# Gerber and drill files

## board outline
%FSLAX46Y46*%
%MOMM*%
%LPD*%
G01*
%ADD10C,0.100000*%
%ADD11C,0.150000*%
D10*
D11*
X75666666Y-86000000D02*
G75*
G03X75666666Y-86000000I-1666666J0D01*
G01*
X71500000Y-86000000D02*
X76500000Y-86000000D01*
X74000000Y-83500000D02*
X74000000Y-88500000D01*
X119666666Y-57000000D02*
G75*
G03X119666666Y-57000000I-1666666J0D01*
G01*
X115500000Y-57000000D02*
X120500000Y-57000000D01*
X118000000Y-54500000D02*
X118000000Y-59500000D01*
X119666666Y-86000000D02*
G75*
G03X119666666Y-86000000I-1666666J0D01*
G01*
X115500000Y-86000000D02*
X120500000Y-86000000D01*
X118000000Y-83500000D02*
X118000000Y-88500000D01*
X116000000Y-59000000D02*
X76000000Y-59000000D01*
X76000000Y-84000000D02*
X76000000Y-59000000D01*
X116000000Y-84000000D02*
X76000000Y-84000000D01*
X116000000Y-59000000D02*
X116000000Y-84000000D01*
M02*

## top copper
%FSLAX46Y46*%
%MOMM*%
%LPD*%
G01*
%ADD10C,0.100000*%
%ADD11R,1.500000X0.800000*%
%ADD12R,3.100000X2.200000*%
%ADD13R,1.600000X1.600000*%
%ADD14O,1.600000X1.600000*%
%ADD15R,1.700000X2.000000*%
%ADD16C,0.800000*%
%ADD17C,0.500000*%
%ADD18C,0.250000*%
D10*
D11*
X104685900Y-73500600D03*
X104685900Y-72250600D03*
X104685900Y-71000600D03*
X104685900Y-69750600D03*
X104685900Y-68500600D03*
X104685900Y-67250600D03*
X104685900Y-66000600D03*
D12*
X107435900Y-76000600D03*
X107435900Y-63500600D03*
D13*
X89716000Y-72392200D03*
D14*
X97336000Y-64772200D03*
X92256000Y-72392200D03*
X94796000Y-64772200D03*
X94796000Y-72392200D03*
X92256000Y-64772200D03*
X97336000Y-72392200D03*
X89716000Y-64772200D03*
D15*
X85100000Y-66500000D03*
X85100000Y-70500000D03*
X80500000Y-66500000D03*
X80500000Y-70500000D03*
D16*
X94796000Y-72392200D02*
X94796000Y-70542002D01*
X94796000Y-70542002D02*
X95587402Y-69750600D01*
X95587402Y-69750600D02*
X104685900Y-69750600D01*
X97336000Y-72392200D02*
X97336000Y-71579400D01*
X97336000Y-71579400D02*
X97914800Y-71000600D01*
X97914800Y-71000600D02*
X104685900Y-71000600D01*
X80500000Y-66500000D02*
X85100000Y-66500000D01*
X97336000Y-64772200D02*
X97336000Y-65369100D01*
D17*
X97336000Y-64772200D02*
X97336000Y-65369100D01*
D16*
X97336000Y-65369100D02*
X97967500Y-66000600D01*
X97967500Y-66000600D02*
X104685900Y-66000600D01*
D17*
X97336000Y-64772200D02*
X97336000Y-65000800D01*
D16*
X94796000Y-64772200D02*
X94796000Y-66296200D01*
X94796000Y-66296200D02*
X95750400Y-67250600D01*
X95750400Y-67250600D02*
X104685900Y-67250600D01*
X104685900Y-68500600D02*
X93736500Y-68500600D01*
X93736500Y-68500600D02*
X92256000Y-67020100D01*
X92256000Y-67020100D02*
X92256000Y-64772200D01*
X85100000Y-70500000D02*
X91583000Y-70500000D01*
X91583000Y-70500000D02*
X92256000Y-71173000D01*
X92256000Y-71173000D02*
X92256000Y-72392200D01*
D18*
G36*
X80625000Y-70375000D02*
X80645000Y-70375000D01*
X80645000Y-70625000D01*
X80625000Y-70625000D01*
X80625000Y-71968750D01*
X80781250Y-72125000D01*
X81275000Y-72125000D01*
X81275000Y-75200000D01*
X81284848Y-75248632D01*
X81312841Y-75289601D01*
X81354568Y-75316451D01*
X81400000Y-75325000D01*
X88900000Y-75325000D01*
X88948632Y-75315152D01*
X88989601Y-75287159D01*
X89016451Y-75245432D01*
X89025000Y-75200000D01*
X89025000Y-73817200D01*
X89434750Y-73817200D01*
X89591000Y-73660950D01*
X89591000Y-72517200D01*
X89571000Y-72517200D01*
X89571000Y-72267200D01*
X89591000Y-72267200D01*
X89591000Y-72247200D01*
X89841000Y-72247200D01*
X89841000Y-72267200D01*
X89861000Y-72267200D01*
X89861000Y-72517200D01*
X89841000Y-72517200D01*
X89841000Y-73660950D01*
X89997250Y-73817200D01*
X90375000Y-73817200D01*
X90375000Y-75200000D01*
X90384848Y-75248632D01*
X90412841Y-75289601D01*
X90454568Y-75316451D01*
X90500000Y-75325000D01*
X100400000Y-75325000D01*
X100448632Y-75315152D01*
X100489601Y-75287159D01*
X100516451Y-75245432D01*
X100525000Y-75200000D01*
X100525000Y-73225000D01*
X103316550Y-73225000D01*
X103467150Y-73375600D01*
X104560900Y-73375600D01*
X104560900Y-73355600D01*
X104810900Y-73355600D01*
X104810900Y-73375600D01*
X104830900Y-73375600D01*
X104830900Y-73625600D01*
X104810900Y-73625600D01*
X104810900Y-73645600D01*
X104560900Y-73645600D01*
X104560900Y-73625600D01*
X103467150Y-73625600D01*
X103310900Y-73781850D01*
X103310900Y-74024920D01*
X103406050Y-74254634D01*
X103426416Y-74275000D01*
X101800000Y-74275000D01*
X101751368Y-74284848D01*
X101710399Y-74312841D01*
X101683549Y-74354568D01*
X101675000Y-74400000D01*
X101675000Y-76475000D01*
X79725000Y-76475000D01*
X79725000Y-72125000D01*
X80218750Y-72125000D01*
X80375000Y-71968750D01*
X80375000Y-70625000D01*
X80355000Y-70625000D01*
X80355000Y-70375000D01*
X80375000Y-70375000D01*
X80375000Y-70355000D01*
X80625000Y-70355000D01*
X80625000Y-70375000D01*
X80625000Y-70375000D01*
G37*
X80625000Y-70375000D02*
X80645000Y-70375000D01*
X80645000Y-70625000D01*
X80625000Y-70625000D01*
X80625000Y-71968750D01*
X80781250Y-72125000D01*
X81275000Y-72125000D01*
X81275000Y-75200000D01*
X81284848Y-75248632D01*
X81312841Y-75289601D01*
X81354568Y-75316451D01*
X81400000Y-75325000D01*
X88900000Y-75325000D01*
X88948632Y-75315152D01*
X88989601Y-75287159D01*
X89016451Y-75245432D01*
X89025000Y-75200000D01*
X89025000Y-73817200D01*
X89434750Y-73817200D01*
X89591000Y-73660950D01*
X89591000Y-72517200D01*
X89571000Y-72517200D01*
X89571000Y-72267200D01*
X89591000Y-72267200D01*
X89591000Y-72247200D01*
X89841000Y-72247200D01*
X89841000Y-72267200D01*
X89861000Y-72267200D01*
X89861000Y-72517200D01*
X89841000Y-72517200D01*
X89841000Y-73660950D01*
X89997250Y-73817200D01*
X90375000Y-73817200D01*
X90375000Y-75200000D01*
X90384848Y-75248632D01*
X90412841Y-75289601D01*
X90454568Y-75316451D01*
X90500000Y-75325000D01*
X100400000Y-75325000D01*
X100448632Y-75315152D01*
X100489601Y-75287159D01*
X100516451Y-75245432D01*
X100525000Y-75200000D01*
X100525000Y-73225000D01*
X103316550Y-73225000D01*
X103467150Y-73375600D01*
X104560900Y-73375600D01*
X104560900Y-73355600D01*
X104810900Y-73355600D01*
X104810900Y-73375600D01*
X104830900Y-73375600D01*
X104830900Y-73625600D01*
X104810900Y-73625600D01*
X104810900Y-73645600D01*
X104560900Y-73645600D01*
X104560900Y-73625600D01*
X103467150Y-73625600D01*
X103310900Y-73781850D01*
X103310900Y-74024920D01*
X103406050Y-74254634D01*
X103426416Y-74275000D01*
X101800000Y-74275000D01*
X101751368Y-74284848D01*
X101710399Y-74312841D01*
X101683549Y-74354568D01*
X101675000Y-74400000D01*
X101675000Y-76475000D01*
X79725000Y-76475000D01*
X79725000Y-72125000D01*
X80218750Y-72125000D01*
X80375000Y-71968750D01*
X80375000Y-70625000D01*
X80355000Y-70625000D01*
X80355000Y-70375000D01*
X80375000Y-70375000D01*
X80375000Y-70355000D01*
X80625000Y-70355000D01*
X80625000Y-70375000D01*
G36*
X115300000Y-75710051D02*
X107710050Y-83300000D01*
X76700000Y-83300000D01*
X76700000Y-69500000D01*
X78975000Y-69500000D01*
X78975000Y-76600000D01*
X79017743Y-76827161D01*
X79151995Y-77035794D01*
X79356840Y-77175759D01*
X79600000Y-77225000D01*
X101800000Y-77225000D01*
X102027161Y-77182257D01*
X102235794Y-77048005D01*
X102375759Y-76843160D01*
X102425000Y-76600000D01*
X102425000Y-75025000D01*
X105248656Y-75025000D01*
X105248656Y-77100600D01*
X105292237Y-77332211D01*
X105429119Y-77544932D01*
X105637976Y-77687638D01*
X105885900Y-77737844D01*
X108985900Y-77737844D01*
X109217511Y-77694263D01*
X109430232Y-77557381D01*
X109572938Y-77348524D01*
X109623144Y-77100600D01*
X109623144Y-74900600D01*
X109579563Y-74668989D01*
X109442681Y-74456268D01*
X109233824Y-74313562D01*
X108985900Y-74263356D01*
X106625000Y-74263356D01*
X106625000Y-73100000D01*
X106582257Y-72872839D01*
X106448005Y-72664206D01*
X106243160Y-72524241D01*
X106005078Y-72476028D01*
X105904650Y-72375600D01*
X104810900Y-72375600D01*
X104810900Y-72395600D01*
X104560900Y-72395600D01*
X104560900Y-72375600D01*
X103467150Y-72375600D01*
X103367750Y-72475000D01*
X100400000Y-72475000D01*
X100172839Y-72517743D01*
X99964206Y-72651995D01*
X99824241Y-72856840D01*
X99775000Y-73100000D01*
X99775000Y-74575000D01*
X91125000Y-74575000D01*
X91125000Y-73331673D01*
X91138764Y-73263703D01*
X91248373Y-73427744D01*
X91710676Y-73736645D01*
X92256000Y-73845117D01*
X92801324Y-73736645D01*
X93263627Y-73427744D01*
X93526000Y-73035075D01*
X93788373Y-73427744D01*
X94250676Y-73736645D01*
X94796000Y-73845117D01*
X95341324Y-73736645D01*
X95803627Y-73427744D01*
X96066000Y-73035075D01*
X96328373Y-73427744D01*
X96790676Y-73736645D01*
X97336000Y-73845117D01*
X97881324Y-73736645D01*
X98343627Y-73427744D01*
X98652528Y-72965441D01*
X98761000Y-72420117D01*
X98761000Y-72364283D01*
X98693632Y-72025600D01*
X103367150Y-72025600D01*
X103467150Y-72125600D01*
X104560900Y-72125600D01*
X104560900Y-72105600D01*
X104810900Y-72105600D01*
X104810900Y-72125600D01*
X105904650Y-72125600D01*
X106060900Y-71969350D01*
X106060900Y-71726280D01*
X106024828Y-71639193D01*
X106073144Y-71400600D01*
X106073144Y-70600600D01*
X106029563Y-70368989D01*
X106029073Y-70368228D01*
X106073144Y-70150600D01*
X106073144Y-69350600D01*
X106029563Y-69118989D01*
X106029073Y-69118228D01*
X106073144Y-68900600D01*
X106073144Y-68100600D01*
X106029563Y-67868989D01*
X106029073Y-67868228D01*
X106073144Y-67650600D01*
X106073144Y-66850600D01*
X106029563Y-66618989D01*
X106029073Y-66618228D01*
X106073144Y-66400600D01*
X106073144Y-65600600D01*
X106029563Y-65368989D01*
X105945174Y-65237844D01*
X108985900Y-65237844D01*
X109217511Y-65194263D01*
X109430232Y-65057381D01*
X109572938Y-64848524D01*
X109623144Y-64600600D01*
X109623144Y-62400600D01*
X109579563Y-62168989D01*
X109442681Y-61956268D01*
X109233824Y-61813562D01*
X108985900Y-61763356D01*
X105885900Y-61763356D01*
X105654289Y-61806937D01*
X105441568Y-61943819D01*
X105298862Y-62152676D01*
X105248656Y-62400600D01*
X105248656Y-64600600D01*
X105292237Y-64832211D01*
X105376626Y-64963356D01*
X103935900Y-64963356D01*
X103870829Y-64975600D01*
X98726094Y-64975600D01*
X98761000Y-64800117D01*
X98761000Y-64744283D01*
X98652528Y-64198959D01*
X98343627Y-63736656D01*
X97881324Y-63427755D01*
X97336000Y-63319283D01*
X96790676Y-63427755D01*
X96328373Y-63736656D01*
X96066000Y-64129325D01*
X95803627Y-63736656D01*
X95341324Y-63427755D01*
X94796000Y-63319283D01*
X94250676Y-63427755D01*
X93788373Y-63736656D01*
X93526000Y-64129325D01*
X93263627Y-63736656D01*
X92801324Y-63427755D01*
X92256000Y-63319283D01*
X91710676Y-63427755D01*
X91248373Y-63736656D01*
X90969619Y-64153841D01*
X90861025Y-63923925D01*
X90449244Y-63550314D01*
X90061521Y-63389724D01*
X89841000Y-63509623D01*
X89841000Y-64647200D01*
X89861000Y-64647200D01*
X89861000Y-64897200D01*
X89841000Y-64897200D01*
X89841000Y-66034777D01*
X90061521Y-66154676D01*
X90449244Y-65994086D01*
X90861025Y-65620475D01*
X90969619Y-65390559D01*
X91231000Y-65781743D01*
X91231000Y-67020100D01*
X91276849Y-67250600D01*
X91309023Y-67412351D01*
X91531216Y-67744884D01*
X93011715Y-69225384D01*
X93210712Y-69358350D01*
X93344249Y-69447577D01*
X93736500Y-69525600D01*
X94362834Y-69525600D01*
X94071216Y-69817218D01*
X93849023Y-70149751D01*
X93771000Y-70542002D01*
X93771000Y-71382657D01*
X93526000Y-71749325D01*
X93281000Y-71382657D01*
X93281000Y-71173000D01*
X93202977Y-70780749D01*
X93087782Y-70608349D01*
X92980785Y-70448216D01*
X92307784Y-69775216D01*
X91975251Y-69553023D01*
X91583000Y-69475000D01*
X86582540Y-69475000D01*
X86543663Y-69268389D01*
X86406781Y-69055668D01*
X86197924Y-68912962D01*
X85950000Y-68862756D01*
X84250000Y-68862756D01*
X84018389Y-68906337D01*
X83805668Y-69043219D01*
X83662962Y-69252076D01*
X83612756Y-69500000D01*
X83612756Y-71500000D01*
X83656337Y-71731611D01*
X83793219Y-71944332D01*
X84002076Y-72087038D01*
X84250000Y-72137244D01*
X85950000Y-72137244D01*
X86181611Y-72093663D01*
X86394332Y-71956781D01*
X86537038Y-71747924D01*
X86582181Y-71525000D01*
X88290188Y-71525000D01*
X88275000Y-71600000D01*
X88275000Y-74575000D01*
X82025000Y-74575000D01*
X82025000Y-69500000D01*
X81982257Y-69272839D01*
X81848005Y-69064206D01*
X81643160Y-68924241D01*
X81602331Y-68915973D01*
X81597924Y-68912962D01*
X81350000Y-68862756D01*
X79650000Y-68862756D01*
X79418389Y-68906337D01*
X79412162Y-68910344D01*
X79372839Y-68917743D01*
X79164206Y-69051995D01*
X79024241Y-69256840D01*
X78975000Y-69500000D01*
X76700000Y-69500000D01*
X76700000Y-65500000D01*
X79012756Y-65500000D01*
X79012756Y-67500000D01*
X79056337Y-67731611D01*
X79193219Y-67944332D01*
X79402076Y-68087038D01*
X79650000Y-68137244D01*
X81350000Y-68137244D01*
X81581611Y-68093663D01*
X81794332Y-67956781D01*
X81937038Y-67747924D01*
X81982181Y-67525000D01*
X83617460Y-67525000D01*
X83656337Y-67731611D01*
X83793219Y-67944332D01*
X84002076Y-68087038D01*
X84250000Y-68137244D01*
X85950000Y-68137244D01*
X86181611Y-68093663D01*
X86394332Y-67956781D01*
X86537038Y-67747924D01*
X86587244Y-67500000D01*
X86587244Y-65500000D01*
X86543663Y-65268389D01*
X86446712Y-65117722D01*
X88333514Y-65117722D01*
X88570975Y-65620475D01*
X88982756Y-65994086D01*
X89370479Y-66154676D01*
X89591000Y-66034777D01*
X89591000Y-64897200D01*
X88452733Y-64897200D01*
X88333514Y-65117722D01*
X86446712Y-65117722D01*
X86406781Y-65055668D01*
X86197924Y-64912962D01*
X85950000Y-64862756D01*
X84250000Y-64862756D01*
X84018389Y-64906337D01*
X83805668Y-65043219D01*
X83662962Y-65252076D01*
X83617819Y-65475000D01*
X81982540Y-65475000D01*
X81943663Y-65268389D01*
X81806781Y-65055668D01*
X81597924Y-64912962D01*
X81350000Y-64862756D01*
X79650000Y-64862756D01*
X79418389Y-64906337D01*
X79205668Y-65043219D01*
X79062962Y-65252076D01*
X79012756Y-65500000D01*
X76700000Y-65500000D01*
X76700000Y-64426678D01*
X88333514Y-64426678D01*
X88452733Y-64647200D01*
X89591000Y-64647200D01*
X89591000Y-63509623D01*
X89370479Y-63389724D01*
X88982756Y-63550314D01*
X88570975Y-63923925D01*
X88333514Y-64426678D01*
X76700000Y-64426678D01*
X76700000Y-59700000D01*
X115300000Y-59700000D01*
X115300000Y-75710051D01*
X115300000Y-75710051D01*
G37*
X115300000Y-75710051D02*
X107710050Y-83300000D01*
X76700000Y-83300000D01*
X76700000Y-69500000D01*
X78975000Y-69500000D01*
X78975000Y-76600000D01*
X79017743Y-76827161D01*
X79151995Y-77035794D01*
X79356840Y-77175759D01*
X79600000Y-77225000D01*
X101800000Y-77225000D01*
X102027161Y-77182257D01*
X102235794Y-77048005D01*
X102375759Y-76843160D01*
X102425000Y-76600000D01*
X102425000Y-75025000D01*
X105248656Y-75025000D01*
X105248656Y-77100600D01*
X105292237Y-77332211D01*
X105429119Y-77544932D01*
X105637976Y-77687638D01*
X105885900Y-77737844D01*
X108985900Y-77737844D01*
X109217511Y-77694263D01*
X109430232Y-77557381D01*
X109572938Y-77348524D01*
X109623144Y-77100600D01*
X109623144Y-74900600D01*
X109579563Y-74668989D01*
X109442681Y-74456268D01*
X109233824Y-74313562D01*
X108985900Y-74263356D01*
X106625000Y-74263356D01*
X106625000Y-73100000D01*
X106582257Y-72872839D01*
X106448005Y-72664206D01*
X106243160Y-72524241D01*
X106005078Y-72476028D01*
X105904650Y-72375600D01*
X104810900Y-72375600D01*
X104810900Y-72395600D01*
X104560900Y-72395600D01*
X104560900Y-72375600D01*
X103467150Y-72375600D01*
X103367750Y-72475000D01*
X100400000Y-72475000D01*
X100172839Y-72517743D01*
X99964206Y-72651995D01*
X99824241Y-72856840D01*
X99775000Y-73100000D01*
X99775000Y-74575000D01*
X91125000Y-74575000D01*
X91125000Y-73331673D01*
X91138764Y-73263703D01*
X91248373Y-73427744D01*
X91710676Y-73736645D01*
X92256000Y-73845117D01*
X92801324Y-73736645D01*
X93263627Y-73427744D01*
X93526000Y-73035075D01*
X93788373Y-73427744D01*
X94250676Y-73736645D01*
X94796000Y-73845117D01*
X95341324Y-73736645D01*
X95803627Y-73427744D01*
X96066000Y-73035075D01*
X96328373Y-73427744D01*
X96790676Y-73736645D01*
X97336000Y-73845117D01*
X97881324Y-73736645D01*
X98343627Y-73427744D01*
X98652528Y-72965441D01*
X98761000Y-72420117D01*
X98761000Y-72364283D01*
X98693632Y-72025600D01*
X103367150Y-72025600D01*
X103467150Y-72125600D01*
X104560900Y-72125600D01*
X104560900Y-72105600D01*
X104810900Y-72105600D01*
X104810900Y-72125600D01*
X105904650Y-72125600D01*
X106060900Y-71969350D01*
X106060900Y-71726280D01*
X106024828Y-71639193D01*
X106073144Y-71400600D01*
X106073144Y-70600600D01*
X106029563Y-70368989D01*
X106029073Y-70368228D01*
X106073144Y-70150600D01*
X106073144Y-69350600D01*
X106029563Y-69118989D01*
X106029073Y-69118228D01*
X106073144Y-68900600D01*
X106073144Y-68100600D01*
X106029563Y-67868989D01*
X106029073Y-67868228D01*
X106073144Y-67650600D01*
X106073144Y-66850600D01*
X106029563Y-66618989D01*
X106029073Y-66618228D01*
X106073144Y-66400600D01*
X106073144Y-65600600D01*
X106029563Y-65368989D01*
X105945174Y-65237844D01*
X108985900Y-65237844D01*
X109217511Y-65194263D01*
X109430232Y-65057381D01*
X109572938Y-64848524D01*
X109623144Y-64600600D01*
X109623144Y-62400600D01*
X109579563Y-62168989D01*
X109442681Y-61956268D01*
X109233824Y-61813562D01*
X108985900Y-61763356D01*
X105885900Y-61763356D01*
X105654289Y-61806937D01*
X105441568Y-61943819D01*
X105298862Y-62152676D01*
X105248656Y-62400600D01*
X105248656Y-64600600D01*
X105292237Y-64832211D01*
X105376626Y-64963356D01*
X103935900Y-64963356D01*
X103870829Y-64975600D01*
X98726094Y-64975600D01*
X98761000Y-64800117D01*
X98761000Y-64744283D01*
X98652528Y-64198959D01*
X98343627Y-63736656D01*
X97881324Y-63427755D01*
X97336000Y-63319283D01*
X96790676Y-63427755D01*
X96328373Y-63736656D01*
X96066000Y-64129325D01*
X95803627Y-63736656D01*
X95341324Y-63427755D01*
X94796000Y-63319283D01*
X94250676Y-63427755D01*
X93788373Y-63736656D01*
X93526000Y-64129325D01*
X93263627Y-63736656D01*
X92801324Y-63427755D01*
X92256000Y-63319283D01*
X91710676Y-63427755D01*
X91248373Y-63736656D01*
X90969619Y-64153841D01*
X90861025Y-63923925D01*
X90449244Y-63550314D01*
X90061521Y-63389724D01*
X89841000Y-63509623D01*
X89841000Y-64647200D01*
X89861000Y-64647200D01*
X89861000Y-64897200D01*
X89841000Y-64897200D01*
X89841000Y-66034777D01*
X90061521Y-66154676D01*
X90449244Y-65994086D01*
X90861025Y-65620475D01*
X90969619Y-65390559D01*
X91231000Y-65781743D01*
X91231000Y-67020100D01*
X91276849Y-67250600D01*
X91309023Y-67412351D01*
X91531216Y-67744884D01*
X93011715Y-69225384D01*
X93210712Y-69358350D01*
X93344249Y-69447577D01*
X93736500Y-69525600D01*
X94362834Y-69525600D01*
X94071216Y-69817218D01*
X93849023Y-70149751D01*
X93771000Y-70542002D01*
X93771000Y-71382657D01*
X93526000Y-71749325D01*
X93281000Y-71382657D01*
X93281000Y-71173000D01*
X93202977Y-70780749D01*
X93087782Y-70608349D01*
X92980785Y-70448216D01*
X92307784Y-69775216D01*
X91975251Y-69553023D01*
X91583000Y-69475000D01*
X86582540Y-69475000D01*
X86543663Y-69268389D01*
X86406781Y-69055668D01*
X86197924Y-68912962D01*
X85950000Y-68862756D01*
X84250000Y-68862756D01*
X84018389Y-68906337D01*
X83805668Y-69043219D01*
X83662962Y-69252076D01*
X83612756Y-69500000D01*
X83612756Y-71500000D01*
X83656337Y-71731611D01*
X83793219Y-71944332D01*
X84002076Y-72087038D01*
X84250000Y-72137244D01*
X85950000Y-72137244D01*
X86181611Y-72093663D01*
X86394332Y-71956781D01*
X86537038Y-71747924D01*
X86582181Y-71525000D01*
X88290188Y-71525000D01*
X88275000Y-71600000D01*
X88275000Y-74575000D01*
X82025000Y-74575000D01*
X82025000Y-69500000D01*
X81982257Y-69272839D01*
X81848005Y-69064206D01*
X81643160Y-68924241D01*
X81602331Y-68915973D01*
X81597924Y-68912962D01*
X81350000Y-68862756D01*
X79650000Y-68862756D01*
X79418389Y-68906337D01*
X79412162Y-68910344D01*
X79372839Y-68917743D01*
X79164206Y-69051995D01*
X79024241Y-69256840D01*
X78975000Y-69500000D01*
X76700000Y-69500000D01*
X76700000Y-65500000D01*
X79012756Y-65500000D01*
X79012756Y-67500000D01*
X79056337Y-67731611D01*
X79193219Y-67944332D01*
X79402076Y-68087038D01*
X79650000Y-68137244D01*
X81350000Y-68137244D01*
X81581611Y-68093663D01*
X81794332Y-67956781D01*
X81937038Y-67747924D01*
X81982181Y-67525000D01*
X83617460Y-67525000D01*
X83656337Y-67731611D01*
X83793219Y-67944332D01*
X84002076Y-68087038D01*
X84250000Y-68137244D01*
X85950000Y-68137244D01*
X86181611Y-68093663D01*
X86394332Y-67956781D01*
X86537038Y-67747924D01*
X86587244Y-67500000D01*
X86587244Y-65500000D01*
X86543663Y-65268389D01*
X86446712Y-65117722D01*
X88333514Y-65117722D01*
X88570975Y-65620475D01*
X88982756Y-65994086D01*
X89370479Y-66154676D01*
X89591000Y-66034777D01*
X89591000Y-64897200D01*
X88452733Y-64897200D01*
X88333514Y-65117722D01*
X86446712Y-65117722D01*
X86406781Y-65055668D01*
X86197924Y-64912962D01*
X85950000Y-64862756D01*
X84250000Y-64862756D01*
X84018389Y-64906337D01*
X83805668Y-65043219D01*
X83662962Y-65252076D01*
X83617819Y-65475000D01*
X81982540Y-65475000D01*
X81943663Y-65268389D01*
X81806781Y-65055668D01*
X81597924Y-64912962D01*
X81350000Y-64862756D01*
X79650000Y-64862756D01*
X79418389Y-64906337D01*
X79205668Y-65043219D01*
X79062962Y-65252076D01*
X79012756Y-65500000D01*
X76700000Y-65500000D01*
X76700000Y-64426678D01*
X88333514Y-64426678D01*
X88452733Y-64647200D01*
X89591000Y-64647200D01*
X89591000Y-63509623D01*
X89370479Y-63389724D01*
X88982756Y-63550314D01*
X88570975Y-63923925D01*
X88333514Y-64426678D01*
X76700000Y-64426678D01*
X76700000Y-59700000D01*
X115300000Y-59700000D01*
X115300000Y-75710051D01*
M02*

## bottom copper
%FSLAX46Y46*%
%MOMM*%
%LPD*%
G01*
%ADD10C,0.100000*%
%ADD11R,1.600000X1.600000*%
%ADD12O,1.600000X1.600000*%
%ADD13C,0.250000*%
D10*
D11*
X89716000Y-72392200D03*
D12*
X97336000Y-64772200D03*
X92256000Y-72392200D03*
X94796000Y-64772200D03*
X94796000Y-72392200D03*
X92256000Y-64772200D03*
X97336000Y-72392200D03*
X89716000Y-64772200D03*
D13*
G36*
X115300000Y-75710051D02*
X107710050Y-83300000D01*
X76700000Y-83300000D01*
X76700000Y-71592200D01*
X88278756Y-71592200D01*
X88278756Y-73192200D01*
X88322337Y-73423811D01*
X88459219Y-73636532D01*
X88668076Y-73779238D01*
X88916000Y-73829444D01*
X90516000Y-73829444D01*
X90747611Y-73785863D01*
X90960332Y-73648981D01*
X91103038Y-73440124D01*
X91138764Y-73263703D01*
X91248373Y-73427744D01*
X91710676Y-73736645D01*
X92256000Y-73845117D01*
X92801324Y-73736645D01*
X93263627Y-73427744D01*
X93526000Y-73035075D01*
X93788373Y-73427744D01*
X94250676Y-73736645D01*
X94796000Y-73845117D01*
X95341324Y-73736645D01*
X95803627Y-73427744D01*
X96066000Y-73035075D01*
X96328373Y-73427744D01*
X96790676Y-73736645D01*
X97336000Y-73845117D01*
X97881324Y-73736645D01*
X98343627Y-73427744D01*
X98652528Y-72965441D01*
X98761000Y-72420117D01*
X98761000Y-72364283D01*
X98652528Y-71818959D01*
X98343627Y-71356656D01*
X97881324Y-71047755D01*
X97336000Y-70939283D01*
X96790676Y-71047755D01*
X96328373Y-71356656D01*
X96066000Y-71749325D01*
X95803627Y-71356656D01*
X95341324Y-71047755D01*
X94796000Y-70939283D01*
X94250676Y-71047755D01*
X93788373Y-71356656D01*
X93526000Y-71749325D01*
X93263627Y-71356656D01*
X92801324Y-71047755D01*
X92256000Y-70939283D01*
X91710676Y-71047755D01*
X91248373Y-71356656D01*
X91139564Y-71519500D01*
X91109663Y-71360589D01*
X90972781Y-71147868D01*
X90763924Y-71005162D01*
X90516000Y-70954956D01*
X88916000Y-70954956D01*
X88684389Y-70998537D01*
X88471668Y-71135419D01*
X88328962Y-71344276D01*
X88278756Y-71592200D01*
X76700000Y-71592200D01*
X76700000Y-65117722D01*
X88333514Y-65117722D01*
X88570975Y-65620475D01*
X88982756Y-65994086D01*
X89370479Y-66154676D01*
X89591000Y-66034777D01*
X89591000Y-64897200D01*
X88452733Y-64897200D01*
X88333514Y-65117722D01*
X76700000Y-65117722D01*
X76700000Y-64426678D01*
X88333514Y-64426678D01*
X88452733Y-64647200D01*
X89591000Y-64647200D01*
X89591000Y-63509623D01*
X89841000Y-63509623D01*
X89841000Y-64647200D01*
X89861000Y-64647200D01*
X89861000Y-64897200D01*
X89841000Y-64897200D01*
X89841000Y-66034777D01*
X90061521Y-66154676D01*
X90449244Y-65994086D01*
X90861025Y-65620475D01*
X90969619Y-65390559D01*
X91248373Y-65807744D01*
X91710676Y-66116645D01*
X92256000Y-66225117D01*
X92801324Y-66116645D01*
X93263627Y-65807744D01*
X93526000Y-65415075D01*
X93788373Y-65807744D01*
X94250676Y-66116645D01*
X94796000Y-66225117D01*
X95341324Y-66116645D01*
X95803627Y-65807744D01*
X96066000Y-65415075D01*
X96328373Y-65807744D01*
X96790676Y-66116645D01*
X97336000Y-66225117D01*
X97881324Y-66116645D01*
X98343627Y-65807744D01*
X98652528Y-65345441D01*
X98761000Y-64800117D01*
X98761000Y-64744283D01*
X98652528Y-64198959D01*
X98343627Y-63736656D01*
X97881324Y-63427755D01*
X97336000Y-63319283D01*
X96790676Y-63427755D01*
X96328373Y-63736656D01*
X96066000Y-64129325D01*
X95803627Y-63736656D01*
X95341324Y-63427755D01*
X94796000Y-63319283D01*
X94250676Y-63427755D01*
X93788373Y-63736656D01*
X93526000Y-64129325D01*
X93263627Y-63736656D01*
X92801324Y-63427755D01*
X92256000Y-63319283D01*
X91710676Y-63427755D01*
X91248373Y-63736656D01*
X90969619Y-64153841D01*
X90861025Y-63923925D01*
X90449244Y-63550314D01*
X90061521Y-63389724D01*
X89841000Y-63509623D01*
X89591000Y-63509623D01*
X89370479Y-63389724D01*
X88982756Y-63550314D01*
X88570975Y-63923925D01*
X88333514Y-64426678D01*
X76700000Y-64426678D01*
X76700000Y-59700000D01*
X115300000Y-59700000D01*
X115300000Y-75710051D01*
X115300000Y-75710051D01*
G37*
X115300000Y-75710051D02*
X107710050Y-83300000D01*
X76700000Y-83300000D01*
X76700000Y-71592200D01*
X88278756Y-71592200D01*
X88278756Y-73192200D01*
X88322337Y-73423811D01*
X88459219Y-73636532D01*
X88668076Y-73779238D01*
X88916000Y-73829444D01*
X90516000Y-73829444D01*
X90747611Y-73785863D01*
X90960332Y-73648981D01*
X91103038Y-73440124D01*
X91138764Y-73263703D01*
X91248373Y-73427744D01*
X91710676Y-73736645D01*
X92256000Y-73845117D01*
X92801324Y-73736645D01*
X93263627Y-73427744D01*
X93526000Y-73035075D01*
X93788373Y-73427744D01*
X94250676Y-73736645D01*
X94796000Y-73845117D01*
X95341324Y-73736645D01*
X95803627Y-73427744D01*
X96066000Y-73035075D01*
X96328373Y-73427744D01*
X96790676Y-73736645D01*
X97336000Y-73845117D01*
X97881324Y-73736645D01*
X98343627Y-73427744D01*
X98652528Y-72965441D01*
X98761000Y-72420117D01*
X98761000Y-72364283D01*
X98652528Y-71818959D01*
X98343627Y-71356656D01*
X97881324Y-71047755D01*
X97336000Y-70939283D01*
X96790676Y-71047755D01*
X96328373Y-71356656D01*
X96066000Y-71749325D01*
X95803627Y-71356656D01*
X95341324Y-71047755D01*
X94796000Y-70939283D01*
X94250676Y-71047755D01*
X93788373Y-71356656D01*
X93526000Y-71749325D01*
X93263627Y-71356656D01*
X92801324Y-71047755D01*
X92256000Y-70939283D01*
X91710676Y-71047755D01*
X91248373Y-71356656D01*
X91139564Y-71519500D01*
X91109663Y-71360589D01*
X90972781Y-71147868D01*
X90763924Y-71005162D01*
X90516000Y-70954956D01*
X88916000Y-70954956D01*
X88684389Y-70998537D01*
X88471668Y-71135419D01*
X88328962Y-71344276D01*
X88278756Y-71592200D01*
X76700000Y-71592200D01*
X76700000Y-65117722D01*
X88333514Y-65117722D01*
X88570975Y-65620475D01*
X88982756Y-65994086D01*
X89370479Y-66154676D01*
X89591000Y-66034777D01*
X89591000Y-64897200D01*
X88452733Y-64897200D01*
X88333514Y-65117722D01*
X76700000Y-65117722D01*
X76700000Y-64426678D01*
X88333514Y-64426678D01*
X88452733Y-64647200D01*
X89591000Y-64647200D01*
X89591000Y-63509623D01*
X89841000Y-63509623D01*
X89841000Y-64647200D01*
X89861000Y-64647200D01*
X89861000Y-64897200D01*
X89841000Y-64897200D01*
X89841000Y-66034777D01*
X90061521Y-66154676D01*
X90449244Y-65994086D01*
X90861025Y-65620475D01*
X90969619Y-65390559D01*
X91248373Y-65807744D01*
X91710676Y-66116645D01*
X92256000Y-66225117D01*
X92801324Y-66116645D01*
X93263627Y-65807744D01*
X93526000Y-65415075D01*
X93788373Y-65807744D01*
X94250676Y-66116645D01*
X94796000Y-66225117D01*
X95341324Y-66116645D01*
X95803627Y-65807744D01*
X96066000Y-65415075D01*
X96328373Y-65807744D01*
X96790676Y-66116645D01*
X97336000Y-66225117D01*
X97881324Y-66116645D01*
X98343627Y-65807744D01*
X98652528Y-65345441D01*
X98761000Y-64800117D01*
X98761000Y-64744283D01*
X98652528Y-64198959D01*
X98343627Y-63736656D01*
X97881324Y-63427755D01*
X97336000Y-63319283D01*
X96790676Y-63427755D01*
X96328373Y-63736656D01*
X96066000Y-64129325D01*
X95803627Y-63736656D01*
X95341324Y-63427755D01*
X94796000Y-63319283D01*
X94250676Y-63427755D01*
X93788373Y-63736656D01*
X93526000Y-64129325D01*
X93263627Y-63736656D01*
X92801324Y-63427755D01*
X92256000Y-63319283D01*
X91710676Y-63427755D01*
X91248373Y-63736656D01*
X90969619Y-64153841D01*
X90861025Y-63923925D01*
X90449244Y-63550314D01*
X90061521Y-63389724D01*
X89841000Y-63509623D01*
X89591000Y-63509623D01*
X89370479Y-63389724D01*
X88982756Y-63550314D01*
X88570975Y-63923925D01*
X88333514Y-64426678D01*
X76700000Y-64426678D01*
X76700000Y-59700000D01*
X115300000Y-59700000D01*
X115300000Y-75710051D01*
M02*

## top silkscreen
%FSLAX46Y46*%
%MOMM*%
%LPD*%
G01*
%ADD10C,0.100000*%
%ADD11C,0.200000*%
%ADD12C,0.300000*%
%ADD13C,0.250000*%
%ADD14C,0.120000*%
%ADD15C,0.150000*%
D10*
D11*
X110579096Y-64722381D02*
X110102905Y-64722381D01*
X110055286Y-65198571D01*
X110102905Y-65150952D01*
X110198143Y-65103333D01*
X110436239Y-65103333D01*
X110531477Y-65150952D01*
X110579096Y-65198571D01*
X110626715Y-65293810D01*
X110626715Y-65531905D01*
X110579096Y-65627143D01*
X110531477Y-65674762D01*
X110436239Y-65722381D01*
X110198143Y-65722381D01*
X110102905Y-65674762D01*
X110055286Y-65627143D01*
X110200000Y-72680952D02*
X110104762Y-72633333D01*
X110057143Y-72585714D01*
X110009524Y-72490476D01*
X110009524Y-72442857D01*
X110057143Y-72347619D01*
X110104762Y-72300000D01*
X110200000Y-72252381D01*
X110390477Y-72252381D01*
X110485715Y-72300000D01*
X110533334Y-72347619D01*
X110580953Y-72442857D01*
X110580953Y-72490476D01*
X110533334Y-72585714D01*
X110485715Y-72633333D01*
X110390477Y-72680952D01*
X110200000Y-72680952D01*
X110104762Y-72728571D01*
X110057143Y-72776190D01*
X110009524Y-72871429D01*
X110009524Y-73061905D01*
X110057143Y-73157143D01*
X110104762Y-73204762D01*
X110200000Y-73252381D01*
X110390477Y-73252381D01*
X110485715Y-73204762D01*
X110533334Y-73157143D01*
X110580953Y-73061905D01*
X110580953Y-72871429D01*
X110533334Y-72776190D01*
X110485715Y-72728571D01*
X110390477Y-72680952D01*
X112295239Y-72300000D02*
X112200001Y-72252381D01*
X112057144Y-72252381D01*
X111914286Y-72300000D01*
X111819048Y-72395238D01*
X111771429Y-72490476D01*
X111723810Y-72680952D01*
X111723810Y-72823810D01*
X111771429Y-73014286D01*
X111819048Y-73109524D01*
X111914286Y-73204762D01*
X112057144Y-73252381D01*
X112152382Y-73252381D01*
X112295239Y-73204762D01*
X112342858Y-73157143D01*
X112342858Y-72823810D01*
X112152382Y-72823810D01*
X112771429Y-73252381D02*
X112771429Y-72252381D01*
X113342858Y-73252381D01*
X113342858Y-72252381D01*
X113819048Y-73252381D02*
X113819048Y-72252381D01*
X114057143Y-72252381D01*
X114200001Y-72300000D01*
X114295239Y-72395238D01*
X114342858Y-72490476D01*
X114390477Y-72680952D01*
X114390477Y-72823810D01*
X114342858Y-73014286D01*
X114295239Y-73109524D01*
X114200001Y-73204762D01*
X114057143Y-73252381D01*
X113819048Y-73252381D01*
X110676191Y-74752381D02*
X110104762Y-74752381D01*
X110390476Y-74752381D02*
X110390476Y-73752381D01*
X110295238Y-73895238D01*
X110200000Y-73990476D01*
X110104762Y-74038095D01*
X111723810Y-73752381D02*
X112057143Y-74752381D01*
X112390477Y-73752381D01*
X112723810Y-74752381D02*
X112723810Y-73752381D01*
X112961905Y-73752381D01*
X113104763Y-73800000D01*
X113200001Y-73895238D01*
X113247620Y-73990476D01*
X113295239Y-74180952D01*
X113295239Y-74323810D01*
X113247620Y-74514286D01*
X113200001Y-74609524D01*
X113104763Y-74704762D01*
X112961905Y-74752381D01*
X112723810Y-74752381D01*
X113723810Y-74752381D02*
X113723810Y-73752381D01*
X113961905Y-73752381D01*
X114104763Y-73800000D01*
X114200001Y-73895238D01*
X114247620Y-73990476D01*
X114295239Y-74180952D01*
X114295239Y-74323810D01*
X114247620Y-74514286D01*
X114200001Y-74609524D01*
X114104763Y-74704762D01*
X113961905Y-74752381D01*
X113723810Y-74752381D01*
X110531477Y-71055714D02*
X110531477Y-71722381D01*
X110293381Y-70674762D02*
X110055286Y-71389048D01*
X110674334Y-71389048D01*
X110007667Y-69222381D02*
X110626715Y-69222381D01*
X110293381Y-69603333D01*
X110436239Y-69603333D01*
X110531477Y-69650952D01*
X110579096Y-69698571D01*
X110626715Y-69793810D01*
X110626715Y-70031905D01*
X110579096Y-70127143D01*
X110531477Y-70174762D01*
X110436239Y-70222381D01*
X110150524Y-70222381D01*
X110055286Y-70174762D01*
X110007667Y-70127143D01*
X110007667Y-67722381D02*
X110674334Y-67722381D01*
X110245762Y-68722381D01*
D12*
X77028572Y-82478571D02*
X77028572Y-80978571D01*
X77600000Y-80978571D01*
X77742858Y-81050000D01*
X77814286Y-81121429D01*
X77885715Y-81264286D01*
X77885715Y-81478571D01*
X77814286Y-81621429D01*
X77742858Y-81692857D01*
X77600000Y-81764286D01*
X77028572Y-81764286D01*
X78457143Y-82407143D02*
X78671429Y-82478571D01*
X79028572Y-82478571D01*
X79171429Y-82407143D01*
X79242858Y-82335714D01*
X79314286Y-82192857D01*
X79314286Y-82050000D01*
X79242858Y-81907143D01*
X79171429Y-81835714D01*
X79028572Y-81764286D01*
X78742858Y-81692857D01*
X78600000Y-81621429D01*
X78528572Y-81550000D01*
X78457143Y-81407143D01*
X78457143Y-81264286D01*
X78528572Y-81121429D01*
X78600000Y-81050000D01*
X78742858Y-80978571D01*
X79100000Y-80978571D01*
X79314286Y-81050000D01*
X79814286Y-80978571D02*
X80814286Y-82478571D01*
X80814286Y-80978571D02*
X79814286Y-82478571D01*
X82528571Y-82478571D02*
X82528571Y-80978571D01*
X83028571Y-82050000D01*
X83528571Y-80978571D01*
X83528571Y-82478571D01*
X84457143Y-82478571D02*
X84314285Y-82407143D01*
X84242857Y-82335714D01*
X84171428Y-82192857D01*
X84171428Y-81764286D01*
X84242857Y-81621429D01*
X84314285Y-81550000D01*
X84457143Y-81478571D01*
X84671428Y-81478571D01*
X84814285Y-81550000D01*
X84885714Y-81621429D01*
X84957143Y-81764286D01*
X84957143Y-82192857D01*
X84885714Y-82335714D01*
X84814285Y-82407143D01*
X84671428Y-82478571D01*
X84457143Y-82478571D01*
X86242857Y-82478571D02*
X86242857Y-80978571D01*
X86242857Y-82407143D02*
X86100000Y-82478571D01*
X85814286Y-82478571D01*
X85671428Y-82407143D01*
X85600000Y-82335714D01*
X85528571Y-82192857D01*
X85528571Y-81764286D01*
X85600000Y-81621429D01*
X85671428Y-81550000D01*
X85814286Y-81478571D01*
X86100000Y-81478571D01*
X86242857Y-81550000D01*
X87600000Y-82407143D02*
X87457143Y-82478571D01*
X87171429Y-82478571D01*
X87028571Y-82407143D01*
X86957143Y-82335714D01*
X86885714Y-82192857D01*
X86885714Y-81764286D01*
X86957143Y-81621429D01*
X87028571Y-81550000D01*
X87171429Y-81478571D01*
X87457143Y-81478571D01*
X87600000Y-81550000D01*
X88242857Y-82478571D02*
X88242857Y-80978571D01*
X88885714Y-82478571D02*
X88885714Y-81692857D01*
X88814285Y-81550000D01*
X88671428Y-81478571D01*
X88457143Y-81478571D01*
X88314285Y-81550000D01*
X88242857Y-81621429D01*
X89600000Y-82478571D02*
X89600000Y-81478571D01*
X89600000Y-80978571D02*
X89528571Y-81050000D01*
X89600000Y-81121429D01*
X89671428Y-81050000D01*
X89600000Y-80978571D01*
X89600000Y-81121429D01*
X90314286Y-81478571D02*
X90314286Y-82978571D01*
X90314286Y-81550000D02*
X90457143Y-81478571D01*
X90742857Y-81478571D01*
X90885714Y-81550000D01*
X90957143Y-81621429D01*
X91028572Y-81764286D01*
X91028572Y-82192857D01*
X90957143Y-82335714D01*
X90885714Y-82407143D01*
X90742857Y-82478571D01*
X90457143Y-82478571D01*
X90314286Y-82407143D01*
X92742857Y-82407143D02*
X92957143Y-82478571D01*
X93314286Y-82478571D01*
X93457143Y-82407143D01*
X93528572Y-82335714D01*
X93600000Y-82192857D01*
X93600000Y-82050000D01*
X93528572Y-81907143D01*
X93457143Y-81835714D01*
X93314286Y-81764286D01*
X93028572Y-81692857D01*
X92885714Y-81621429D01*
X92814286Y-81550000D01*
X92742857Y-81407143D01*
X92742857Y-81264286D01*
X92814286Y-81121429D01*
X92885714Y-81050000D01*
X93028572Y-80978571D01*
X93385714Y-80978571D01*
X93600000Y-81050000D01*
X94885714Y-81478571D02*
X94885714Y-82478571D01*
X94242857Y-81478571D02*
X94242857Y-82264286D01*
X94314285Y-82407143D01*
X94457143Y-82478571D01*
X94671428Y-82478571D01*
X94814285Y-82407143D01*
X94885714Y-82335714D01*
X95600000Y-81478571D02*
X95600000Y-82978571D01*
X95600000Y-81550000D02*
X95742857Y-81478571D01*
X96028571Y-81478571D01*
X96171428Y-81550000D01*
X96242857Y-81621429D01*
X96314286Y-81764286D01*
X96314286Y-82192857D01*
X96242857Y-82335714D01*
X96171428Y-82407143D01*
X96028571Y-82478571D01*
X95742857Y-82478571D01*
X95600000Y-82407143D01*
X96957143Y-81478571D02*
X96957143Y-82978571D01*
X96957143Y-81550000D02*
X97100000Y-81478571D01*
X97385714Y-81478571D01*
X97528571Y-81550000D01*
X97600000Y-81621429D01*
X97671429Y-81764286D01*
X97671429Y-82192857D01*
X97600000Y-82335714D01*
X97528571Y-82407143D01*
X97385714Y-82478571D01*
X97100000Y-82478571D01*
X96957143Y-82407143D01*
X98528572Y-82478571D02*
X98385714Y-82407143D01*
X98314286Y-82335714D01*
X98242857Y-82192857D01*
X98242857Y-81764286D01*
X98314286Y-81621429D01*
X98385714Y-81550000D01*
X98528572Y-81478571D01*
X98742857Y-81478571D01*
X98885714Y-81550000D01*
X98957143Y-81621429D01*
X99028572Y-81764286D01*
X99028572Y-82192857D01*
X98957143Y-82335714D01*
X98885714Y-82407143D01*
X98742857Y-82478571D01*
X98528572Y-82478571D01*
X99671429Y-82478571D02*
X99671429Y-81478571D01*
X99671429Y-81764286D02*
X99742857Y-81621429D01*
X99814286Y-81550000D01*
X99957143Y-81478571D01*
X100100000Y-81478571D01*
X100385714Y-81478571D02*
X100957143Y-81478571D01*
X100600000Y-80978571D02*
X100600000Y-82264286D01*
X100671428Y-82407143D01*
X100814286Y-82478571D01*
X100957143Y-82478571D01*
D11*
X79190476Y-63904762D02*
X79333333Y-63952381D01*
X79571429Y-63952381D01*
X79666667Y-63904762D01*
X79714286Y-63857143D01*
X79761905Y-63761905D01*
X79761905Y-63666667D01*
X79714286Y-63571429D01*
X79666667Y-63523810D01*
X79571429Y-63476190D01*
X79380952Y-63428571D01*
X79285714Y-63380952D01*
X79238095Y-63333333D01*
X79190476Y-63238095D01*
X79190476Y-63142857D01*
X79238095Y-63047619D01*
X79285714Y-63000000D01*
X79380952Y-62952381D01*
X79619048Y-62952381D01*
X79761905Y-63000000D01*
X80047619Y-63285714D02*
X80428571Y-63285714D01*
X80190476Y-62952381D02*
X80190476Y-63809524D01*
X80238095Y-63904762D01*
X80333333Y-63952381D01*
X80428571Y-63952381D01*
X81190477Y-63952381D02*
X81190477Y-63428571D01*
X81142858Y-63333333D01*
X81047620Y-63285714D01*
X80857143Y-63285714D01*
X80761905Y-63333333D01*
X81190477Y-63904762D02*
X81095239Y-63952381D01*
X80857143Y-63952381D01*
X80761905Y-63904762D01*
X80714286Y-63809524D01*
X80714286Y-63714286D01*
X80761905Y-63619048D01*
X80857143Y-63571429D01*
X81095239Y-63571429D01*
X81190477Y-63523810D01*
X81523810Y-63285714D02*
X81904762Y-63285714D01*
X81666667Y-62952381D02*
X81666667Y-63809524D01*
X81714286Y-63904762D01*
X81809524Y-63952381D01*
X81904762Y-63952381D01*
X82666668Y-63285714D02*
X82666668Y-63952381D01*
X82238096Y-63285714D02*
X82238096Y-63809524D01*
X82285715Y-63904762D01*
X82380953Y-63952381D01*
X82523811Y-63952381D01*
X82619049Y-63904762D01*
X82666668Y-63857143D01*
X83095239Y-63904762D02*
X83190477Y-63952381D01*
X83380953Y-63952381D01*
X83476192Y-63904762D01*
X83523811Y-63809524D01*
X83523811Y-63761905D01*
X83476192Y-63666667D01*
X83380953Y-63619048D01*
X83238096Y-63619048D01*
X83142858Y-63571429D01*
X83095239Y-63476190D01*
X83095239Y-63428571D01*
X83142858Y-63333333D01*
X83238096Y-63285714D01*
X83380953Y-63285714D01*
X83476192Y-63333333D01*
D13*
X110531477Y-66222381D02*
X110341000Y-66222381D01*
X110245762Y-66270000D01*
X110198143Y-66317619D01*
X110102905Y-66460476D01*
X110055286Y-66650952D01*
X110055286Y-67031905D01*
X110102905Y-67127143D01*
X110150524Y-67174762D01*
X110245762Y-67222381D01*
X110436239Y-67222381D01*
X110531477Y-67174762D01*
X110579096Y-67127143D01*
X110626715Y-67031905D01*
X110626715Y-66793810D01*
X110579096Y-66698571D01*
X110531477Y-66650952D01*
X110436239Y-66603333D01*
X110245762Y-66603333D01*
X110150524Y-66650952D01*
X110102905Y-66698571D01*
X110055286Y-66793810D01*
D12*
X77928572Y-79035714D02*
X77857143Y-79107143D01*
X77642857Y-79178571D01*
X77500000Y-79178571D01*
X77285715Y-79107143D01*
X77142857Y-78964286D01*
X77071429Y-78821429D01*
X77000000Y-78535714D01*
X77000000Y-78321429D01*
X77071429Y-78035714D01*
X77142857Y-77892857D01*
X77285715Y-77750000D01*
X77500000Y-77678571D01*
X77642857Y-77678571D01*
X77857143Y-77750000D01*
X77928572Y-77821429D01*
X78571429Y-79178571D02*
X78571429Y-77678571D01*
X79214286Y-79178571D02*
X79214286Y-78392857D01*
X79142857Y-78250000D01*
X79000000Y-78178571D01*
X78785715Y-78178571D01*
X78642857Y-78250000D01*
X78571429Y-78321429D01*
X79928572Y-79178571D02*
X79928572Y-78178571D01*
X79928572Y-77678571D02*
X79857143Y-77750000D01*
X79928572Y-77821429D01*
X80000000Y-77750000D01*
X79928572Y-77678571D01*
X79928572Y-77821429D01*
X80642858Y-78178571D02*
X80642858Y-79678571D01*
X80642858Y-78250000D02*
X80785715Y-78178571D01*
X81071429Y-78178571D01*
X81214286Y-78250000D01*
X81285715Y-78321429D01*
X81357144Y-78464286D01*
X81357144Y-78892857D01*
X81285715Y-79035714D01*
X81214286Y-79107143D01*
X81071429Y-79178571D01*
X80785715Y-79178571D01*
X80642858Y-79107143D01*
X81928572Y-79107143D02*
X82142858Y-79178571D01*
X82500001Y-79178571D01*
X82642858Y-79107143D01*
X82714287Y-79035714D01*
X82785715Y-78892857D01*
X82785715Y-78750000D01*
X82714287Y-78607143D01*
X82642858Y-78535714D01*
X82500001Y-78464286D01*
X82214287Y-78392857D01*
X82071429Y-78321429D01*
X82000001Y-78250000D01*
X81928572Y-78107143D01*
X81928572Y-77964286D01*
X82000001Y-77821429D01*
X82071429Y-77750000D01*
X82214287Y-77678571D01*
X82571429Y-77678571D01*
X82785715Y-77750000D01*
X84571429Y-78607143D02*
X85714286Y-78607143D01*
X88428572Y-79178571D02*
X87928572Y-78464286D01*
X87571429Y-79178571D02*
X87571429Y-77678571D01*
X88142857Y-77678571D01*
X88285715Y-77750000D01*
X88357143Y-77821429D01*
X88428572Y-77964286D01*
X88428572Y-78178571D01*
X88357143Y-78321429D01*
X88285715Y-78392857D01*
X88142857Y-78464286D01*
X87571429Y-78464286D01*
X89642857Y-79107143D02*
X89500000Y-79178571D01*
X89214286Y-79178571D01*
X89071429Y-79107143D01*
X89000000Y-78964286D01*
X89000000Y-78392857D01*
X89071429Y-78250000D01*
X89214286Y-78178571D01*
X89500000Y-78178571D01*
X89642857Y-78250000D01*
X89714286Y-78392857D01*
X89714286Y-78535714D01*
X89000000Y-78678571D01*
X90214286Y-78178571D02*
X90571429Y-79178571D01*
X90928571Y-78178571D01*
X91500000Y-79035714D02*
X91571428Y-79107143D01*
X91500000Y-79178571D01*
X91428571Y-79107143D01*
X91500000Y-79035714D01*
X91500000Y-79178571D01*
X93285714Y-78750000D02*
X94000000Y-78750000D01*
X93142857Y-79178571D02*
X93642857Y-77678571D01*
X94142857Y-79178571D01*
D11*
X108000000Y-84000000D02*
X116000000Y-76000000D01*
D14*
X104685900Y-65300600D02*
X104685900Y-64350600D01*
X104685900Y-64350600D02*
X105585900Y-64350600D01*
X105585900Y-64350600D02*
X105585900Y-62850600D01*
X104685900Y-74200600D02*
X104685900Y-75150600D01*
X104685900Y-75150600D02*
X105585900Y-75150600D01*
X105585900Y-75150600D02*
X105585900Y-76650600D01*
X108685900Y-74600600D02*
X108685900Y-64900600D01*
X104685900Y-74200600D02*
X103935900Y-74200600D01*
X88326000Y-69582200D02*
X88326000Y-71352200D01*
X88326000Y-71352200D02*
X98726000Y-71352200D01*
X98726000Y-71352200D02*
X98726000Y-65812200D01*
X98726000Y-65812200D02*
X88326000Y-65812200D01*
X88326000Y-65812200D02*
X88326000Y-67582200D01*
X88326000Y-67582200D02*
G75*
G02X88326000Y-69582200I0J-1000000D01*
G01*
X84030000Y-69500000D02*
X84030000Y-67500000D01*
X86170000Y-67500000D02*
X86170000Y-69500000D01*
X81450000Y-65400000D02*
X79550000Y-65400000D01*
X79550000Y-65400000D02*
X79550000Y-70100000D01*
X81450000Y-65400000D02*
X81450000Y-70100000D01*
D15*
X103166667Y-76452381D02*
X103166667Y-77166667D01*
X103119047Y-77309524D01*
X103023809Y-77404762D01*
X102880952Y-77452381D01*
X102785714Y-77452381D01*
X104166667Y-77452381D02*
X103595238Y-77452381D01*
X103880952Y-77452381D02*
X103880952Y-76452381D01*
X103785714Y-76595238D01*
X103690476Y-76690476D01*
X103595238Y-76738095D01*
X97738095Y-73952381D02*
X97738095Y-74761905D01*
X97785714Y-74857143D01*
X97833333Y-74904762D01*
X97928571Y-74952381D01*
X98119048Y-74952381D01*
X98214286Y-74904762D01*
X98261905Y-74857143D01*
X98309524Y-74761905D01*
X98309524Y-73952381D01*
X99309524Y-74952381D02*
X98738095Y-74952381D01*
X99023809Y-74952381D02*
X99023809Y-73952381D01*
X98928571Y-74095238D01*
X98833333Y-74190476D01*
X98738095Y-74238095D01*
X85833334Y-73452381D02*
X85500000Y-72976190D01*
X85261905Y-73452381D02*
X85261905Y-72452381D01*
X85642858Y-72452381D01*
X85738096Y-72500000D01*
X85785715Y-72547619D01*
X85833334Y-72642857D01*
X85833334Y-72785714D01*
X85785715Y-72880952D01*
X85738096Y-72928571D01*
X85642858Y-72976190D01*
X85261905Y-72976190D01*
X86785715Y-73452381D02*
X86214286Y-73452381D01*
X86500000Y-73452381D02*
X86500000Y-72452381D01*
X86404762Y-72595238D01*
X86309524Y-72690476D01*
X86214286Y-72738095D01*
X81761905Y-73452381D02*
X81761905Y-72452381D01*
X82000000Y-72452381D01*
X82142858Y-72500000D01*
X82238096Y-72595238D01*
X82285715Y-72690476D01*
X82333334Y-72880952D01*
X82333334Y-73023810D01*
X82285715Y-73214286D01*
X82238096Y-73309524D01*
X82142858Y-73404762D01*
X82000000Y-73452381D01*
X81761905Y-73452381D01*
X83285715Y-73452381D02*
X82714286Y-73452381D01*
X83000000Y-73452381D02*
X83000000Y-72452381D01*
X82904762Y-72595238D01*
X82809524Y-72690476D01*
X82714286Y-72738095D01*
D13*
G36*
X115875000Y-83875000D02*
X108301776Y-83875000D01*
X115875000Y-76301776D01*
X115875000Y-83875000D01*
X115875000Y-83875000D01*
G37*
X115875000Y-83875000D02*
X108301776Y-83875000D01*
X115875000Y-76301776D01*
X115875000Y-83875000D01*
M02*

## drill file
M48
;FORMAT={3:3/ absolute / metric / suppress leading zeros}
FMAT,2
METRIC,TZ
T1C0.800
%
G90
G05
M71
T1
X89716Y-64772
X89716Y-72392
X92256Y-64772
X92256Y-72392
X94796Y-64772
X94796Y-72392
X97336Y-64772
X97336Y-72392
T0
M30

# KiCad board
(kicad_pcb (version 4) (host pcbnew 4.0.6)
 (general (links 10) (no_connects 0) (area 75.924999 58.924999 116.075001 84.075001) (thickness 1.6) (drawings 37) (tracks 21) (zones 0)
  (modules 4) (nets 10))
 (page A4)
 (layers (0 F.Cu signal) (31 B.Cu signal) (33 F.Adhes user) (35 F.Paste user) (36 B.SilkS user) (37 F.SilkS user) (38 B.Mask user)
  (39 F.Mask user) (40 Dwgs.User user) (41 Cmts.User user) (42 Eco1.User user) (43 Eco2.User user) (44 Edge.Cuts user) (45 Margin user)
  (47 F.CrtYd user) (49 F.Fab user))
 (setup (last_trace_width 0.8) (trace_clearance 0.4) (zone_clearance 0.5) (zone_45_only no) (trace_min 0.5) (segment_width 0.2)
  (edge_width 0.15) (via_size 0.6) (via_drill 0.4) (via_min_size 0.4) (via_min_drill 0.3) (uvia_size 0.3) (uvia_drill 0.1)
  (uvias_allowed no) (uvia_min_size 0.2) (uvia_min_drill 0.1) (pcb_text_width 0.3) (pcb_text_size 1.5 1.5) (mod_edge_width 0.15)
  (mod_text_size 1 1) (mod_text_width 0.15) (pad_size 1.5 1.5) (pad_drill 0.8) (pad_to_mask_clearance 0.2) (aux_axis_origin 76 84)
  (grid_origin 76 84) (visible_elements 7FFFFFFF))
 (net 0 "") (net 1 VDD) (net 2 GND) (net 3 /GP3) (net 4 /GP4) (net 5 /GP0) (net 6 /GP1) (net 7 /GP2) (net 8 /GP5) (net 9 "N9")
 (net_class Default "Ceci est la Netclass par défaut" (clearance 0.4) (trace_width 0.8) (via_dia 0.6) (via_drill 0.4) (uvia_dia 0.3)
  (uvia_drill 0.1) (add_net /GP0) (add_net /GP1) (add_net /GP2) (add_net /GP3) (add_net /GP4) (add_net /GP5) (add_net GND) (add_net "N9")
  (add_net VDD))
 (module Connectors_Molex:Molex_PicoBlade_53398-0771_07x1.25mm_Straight (layer F.Cu) (at 106.0609 69.7506 90)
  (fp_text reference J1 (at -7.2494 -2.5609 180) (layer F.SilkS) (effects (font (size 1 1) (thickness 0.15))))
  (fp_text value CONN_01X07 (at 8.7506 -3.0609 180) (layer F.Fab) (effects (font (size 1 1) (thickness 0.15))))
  (fp_line (start 4.45 -1.375) (end 5.4 -1.375) (layer F.SilkS) (width 0.12))
  (fp_line (start 5.4 -1.375) (end 5.4 -0.475) (layer F.SilkS) (width 0.12))
  (fp_line (start 5.4 -0.475) (end 6.9 -0.475) (layer F.SilkS) (width 0.12))
  (fp_line (start -4.45 -1.375) (end -5.4 -1.375) (layer F.SilkS) (width 0.12))
  (fp_line (start -5.4 -1.375) (end -5.4 -0.475) (layer F.SilkS) (width 0.12))
  (fp_line (start -5.4 -0.475) (end -6.9 -0.475) (layer F.SilkS) (width 0.12))
  (fp_line (start -4.85 2.625) (end 4.85 2.625) (layer F.SilkS) (width 0.12))
  (fp_line (start -4.45 -1.375) (end -4.45 -2.125) (layer F.SilkS) (width 0.12))
  (pad 1 smd rect (at -3.75 -1.375 90) (size 0.8 1.5) (layers F.Cu F.Paste F.Mask) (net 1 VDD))
  (pad 2 smd rect (at -2.5 -1.375 90) (size 0.8 1.5) (layers F.Cu F.Paste F.Mask) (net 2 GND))
  (pad 3 smd rect (at -1.25 -1.375 90) (size 0.8 1.5) (layers F.Cu F.Paste F.Mask) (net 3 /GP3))
  (pad 4 smd rect (at 0 -1.375 90) (size 0.8 1.5) (layers F.Cu F.Paste F.Mask) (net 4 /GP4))
  (pad 5 smd rect (at 1.25 -1.375 90) (size 0.8 1.5) (layers F.Cu F.Paste F.Mask) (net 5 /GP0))
  (pad 6 smd rect (at 2.5 -1.375 90) (size 0.8 1.5) (layers F.Cu F.Paste F.Mask) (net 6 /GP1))
  (pad 7 smd rect (at 3.75 -1.375 90) (size 0.8 1.5) (layers F.Cu F.Paste F.Mask) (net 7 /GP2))
  (pad "" smd rect (at -6.25 1.375 90) (size 2.2 3.1) (layers F.Cu F.Paste F.Mask))
  (pad "" smd rect (at 6.25 1.375 90) (size 2.2 3.1) (layers F.Cu F.Paste F.Mask)))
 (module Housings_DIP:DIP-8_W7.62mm (layer F.Cu) (at 89.716 72.3922 90)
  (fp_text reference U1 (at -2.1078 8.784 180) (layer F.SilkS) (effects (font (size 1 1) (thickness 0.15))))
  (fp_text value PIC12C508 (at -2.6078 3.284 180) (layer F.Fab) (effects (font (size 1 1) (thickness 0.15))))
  (fp_line (start 2.81 -1.39) (end 1.04 -1.39) (layer F.SilkS) (width 0.12))
  (fp_line (start 1.04 -1.39) (end 1.04 9.01) (layer F.SilkS) (width 0.12))
  (fp_line (start 1.04 9.01) (end 6.58 9.01) (layer F.SilkS) (width 0.12))
  (fp_line (start 6.58 9.01) (end 6.58 -1.39) (layer F.SilkS) (width 0.12))
  (fp_line (start 6.58 -1.39) (end 4.81 -1.39) (layer F.SilkS) (width 0.12))
  (fp_arc (start 3.81 -1.39) (end 2.81 -1.39) (angle -180) (layer F.SilkS) (width 0.12))
  (pad 1 thru_hole rect (at 0 0 90) (size 1.6 1.6) (drill 0.8) (layers *.Cu *.Mask) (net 1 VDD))
  (pad 5 thru_hole oval (at 7.62 7.62 90) (size 1.6 1.6) (drill 0.8) (layers *.Cu *.Mask) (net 7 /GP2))
  (pad 2 thru_hole oval (at 0 2.54 90) (size 1.6 1.6) (drill 0.8) (layers *.Cu *.Mask) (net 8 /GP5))
  (pad 6 thru_hole oval (at 7.62 5.08 90) (size 1.6 1.6) (drill 0.8) (layers *.Cu *.Mask) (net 6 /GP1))
  (pad 3 thru_hole oval (at 0 5.08 90) (size 1.6 1.6) (drill 0.8) (layers *.Cu *.Mask) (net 4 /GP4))
  (pad 7 thru_hole oval (at 7.62 2.54 90) (size 1.6 1.6) (drill 0.8) (layers *.Cu *.Mask) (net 5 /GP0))
  (pad 4 thru_hole oval (at 0 7.62 90) (size 1.6 1.6) (drill 0.8) (layers *.Cu *.Mask) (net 3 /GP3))
  (pad 8 thru_hole oval (at 7.62 0 90) (size 1.6 1.6) (drill 0.8) (layers *.Cu *.Mask) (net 2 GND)))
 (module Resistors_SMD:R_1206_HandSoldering (layer F.Cu) (at 85.1 68.5 270)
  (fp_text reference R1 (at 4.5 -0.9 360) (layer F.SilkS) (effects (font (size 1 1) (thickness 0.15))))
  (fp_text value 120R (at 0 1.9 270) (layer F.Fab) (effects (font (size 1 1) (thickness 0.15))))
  (fp_line (start 1 1.07) (end -1 1.07) (layer F.SilkS) (width 0.12))
  (fp_line (start -1 -1.07) (end 1 -1.07) (layer F.SilkS) (width 0.12))
  (pad 1 smd rect (at -2 0 270) (size 2 1.7) (layers F.Cu F.Paste F.Mask) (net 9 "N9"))
  (pad 2 smd rect (at 2 0 270) (size 2 1.7) (layers F.Cu F.Paste F.Mask) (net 8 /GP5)))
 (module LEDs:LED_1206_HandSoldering (layer F.Cu) (at 80.5 68.5 270)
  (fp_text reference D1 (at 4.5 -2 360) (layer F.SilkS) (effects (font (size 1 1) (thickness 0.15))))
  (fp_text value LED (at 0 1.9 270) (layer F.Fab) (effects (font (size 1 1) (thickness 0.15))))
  (fp_line (start -3.1 -0.95) (end -3.1 0.95) (layer F.SilkS) (width 0.12))
  (fp_line (start -3.1 0.95) (end 1.6 0.95) (layer F.SilkS) (width 0.12))
  (fp_line (start -3.1 -0.95) (end 1.6 -0.95) (layer F.SilkS) (width 0.12))
  (pad 1 smd rect (at -2 0 270) (size 2 1.7) (layers F.Cu F.Paste F.Mask) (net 9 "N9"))
  (pad 2 smd rect (at 2 0 270) (size 2 1.7) (layers F.Cu F.Paste F.Mask) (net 1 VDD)))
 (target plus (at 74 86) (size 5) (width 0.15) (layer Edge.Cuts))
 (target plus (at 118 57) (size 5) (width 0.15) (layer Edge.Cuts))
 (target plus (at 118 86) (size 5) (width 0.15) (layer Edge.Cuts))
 (gr_line (start 116 59) (end 76 59) (angle 90) (layer Edge.Cuts) (width 0.15))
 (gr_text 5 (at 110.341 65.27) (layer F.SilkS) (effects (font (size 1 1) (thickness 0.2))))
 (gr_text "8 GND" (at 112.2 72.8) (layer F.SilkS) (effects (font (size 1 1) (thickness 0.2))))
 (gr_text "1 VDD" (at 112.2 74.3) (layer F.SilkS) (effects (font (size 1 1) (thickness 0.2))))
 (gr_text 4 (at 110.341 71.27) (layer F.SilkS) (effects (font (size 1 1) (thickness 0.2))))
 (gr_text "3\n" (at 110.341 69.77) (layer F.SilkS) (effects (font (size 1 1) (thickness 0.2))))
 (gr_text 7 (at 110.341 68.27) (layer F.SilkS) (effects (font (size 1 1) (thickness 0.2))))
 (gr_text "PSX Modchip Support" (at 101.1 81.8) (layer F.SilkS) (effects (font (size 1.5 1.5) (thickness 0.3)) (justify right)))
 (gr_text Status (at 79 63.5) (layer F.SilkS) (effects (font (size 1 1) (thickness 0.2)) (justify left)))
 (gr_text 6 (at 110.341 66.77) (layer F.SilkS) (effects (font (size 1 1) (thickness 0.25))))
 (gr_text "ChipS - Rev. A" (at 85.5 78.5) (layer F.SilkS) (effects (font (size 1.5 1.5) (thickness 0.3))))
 (gr_line (start 108 84) (end 116 76) (angle 90) (layer F.SilkS) (width 0.2))
 (gr_line (start 76 84) (end 76 59) (angle 90) (layer Edge.Cuts) (width 0.15))
 (gr_line (start 116 84) (end 76 84) (angle 90) (layer Edge.Cuts) (width 0.15))
 (gr_line (start 116 59) (end 116 84) (angle 90) (layer Edge.Cuts) (width 0.15))
 (segment (start 94.796 72.3922) (end 94.796 70.542002) (width 0.8) (layer F.Cu) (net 4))
 (segment (start 94.796 70.542002) (end 95.587402 69.7506) (width 0.8) (layer F.Cu) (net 4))
 (segment (start 95.587402 69.7506) (end 104.6859 69.7506) (width 0.8) (layer F.Cu) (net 4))
 (segment (start 97.336 72.3922) (end 97.336 71.5794) (width 0.8) (layer F.Cu) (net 3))
 (segment (start 97.336 71.5794) (end 97.9148 71.0006) (width 0.8) (layer F.Cu) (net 3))
 (segment (start 97.9148 71.0006) (end 104.6859 71.0006) (width 0.8) (layer F.Cu) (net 3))
 (segment (start 80.5 66.5) (end 85.1 66.5) (width 0.8) (layer F.Cu) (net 9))
 (segment (start 97.336 64.7722) (end 97.336 65.3691) (width 0.8) (layer F.Cu) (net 7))
 (segment (start 97.336 64.7722) (end 97.336 65.3691) (width 0.5) (layer F.Cu) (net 7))
 (segment (start 97.336 65.3691) (end 97.9675 66.0006) (width 0.8) (layer F.Cu) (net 7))
 (segment (start 97.9675 66.0006) (end 104.6859 66.0006) (width 0.8) (layer F.Cu) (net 7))
 (segment (start 97.336 64.7722) (end 97.336 65.0008) (width 0.5) (layer F.Cu) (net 7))
 (segment (start 94.796 64.7722) (end 94.796 66.2962) (width 0.8) (layer F.Cu) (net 6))
 (segment (start 94.796 66.2962) (end 95.7504 67.2506) (width 0.8) (layer F.Cu) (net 6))
 (segment (start 95.7504 67.2506) (end 104.6859 67.2506) (width 0.8) (layer F.Cu) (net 6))
 (segment (start 104.6859 68.5006) (end 93.7365 68.5006) (width 0.8) (layer F.Cu) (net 5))
 (segment (start 93.7365 68.5006) (end 92.256 67.0201) (width 0.8) (layer F.Cu) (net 5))
 (segment (start 92.256 67.0201) (end 92.256 64.7722) (width 0.8) (layer F.Cu) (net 5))
 (segment (start 85.1 70.5) (end 91.583 70.5) (width 0.8) (layer F.Cu) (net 8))
 (segment (start 91.583 70.5) (end 92.256 71.173) (width 0.8) (layer F.Cu) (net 8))
 (segment (start 92.256 71.173) (end 92.256 72.3922) (width 0.8) (layer F.Cu) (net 8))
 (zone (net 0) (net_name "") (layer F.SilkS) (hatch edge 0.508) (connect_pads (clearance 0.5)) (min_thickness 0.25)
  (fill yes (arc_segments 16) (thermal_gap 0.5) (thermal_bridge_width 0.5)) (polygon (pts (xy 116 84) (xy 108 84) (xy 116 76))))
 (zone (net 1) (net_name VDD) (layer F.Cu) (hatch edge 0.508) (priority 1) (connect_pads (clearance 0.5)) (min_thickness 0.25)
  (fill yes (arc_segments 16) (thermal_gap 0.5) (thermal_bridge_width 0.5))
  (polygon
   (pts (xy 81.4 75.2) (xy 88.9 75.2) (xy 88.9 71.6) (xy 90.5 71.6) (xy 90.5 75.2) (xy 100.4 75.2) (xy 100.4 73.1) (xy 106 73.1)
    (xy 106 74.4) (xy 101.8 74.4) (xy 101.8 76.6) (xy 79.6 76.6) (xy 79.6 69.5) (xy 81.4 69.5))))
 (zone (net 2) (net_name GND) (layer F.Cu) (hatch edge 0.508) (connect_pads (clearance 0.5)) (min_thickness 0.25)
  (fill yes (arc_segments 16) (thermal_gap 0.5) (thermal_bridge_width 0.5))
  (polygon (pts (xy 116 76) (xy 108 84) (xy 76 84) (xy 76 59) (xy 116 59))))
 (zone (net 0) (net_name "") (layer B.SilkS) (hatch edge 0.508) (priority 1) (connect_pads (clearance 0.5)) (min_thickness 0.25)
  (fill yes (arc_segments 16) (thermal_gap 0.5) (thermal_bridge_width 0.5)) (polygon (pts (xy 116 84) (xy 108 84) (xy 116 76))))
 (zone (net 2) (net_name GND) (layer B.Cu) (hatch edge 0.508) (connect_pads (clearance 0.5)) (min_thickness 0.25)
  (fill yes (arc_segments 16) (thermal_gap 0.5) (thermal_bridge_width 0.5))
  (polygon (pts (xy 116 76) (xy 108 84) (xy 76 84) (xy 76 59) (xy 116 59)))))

